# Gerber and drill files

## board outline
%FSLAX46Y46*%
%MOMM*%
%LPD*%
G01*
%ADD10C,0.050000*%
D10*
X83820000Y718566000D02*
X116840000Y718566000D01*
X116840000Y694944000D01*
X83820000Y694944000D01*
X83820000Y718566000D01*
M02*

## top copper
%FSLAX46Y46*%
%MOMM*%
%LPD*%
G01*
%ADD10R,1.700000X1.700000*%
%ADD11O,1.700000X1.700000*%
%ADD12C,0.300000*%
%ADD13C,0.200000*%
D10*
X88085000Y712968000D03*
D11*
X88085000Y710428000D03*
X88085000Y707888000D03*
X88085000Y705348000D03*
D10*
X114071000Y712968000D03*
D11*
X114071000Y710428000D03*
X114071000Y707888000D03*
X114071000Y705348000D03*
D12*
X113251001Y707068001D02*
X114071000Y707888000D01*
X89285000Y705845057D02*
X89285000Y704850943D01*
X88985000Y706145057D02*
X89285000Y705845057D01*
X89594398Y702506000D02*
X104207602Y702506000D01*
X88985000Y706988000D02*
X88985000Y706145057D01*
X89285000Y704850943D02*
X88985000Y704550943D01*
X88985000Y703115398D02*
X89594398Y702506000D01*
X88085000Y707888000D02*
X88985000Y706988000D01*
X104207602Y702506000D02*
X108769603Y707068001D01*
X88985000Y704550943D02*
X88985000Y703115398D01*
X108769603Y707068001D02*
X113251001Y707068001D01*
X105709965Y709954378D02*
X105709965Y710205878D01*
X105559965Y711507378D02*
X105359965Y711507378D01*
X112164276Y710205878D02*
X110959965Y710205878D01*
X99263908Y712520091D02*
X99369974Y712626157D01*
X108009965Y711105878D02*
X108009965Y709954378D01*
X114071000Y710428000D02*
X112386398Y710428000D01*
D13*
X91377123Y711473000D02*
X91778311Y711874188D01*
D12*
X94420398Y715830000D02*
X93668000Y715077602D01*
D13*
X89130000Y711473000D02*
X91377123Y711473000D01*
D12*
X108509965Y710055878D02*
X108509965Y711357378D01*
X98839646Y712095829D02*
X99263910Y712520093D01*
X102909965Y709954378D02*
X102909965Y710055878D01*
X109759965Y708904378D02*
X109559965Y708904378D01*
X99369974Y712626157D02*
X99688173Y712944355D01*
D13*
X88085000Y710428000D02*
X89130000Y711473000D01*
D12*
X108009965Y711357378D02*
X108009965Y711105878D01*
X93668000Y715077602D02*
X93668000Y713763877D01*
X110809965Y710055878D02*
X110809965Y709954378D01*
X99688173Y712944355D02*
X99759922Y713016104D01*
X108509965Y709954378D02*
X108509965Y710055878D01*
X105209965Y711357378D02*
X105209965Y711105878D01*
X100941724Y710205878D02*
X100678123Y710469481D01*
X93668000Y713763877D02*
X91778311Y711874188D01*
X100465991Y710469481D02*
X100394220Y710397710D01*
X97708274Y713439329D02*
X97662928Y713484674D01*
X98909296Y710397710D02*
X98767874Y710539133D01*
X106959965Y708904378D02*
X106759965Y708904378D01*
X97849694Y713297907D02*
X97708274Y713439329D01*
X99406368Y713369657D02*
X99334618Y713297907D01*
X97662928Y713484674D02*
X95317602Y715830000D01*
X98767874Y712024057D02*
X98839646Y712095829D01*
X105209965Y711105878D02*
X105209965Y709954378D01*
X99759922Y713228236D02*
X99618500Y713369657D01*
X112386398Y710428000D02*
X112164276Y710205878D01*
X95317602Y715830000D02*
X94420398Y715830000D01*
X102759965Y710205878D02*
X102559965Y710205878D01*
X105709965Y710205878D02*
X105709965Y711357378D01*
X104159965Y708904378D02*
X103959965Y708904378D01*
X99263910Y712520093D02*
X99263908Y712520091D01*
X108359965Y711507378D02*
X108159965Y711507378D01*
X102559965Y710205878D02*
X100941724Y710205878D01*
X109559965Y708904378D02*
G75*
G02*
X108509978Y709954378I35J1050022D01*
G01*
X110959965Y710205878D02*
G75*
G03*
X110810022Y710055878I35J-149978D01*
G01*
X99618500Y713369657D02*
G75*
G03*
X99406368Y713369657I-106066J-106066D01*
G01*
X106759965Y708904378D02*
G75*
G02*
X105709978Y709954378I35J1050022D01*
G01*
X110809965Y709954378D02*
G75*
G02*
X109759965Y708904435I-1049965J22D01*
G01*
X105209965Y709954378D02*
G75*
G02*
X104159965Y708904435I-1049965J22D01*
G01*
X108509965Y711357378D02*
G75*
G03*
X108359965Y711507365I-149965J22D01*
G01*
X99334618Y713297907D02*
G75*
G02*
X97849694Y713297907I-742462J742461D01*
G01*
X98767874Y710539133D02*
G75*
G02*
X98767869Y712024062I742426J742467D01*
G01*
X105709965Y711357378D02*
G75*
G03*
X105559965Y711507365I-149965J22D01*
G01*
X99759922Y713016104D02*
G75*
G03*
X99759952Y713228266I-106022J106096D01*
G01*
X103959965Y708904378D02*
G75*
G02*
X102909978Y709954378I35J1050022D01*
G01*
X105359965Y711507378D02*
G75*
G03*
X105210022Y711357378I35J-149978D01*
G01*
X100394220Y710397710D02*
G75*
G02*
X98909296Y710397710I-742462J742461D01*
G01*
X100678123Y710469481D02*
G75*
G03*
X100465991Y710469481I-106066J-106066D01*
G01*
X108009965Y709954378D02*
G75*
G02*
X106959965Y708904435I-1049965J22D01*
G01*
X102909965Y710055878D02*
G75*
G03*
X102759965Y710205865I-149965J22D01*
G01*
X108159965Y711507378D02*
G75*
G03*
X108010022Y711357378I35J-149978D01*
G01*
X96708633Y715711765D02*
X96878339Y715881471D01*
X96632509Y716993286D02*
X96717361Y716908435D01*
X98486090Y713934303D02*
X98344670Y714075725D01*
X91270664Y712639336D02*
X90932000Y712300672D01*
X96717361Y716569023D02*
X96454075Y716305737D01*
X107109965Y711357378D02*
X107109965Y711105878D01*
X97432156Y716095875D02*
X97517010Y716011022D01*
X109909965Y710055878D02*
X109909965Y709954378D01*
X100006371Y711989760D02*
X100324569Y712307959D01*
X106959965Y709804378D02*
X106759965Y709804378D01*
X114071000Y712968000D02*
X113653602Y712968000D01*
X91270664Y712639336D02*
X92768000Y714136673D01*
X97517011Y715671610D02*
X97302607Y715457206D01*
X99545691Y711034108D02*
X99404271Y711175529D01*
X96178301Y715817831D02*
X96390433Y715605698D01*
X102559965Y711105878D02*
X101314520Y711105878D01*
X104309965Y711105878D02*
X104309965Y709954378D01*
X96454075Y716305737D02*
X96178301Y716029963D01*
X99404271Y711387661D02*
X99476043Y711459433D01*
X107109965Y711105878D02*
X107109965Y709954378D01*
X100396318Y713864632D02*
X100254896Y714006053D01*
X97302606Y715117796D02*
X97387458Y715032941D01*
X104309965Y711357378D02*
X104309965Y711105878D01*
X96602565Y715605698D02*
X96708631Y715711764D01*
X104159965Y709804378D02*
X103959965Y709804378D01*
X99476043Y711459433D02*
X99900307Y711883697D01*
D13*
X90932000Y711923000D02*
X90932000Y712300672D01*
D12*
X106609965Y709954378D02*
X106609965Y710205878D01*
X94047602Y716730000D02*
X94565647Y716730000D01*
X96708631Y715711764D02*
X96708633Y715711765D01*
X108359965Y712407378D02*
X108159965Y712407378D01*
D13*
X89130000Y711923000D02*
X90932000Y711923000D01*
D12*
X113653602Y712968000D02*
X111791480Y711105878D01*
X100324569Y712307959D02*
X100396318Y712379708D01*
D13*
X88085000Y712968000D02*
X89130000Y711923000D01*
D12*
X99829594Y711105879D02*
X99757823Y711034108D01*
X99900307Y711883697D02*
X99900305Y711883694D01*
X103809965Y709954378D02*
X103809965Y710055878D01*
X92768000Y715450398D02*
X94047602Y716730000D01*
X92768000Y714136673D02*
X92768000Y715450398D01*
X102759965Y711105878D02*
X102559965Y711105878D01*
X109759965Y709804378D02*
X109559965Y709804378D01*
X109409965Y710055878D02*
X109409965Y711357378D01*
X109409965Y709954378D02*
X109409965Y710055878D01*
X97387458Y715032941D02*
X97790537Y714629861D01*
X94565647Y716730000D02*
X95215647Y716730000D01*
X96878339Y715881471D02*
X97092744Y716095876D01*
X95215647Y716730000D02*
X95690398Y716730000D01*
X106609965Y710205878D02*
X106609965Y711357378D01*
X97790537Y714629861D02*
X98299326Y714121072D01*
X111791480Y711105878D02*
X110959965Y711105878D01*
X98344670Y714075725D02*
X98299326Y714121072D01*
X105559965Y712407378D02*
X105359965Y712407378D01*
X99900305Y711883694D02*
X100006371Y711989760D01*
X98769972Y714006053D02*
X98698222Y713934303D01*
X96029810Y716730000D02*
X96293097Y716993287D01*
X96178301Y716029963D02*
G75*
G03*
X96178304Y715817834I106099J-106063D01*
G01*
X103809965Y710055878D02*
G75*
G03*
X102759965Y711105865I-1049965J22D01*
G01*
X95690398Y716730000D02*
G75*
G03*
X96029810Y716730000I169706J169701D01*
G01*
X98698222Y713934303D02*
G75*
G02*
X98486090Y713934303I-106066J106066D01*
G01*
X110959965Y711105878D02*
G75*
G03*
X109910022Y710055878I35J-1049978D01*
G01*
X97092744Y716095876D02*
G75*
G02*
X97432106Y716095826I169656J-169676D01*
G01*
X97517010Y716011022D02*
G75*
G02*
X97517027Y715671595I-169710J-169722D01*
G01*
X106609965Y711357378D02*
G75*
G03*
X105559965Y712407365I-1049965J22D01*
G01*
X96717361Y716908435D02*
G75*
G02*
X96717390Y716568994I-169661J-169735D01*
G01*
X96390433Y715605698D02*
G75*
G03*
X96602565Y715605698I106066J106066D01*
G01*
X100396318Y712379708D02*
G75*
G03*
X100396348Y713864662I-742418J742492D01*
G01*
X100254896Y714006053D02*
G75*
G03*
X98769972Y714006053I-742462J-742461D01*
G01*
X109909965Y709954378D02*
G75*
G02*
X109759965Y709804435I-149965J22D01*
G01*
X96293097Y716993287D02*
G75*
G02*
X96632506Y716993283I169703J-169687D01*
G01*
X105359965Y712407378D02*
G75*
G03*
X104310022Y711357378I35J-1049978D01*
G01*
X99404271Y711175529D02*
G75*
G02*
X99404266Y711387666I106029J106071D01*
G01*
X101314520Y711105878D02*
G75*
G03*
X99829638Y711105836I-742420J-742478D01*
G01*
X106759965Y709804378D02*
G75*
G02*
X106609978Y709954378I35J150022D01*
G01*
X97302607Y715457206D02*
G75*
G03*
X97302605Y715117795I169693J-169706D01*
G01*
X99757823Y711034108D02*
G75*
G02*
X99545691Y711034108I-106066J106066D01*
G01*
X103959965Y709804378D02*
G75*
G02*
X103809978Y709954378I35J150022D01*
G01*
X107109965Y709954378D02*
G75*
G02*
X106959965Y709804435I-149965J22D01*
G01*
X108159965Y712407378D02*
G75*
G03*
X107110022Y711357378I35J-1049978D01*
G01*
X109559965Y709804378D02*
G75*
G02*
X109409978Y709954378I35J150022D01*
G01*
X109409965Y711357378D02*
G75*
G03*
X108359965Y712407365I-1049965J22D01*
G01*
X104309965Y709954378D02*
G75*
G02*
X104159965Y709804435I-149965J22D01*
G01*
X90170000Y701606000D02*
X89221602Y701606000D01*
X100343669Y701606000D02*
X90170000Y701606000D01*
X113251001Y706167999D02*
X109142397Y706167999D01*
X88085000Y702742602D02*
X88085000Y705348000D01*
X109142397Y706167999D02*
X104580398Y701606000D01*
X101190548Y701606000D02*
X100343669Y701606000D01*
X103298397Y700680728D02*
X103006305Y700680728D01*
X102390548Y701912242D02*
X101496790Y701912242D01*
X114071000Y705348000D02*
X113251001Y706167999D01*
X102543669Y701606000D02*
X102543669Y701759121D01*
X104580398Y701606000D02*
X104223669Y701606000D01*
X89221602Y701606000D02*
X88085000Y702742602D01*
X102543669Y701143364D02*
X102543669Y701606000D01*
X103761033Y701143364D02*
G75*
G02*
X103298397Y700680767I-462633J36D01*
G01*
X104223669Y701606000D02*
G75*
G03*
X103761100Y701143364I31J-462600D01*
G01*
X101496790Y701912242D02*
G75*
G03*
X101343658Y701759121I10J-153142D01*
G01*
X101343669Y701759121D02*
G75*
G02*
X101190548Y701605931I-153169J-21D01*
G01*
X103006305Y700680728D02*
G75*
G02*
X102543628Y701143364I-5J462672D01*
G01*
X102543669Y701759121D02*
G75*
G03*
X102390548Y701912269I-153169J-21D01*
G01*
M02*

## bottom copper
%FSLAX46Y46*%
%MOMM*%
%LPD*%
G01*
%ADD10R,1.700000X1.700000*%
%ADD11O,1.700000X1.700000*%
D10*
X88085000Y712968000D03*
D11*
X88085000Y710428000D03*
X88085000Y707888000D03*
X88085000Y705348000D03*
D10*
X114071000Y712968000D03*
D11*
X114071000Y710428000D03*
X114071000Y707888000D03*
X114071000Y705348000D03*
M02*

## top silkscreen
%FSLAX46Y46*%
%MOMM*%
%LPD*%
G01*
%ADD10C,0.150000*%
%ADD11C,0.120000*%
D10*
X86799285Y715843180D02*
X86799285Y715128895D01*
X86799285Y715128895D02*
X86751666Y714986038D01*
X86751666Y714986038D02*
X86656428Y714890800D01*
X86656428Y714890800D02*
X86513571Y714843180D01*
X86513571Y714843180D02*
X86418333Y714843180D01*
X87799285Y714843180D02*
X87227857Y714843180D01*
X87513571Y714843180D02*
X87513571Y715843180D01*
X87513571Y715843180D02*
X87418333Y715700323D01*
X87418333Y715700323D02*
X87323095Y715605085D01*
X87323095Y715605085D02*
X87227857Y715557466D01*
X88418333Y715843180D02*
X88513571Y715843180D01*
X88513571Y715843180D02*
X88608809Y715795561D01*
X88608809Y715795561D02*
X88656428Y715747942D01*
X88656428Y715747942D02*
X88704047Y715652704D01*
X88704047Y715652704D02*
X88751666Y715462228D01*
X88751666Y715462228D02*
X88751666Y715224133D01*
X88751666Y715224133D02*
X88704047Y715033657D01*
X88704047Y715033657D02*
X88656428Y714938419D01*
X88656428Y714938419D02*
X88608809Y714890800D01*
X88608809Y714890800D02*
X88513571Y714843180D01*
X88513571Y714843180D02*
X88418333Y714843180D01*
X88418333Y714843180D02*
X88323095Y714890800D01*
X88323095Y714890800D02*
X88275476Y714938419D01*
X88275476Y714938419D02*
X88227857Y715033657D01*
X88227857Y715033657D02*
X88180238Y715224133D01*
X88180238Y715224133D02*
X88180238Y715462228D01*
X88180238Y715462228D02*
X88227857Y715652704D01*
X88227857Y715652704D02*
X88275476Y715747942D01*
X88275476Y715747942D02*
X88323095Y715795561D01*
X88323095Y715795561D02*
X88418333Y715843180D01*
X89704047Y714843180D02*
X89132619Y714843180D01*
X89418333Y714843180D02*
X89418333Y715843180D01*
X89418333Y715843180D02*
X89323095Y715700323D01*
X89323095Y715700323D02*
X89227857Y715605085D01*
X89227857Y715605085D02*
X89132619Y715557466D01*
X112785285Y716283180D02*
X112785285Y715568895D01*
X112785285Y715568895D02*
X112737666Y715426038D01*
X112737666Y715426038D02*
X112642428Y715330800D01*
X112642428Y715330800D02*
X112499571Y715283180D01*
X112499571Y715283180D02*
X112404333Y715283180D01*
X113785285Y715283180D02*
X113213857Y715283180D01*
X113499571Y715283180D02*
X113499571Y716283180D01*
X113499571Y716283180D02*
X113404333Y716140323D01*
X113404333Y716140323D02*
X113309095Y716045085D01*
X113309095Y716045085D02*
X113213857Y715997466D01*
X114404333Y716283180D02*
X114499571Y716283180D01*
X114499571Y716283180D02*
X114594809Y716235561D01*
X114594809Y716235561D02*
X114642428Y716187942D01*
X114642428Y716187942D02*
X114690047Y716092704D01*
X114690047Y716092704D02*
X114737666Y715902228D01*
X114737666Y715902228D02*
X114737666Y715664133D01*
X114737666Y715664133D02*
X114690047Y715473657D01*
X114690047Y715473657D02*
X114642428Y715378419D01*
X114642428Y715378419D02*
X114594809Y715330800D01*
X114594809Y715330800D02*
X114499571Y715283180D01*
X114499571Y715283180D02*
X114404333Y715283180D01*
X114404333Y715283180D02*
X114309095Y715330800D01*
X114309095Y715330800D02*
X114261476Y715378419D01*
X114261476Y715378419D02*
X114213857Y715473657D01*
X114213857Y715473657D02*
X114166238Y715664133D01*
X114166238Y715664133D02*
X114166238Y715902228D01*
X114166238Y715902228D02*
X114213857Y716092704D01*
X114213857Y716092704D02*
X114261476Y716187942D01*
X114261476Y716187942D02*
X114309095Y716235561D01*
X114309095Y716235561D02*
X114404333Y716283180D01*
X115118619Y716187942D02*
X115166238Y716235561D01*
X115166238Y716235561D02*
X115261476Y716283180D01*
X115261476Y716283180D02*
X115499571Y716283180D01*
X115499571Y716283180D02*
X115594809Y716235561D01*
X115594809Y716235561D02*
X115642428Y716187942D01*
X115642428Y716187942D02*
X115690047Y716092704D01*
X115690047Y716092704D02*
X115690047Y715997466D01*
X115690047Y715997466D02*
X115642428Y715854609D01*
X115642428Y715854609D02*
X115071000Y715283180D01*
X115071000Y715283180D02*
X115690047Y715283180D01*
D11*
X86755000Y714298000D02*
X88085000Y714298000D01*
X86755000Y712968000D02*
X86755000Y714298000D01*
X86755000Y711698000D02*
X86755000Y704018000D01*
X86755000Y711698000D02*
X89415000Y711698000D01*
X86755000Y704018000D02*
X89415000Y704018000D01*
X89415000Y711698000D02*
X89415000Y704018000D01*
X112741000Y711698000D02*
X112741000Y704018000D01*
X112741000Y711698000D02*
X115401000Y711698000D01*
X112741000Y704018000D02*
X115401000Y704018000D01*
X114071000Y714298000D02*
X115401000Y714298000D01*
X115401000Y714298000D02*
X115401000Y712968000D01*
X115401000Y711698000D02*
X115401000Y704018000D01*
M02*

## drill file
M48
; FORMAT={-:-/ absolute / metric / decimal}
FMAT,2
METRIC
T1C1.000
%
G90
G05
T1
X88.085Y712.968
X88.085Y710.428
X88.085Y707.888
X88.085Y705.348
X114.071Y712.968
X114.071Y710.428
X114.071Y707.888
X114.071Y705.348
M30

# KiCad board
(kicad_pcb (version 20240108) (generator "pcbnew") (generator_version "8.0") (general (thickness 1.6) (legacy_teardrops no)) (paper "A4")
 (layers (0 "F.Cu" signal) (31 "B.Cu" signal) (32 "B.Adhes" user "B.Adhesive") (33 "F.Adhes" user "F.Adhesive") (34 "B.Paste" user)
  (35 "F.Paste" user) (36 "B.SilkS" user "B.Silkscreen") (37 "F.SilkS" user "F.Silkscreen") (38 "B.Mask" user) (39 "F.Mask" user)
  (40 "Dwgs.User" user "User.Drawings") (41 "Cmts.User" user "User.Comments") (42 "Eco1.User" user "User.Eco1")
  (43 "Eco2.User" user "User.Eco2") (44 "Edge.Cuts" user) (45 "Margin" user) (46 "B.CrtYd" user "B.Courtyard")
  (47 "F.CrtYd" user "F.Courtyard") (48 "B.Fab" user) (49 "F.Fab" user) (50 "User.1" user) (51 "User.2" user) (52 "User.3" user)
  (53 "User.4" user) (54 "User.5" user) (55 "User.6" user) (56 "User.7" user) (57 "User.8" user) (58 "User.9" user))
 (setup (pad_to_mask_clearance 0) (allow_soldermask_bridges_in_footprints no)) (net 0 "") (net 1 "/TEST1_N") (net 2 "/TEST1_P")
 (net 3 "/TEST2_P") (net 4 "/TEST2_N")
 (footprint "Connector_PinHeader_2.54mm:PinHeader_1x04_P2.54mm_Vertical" (layer "F.Cu") (at 88.085 -712.968)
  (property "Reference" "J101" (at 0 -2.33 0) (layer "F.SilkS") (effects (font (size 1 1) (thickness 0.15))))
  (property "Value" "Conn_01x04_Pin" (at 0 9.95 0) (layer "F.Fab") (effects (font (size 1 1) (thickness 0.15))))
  (fp_line (start -1.33 -1.33) (end 0 -1.33) (stroke (width 0.12) (type solid)) (layer "F.SilkS"))
  (fp_line (start -1.33 0) (end -1.33 -1.33) (stroke (width 0.12) (type solid)) (layer "F.SilkS"))
  (fp_line (start -1.33 1.27) (end -1.33 8.95) (stroke (width 0.12) (type solid)) (layer "F.SilkS"))
  (fp_line (start -1.33 1.27) (end 1.33 1.27) (stroke (width 0.12) (type solid)) (layer "F.SilkS"))
  (fp_line (start -1.33 8.95) (end 1.33 8.95) (stroke (width 0.12) (type solid)) (layer "F.SilkS"))
  (fp_line (start 1.33 1.27) (end 1.33 8.95) (stroke (width 0.12) (type solid)) (layer "F.SilkS"))
  (pad "1" thru_hole rect (at 0 0) (size 1.7 1.7) (drill 1) (layers "*.Cu" "*.Mask") (remove_unused_layers no) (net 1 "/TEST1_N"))
  (pad "2" thru_hole oval (at 0 2.54) (size 1.7 1.7) (drill 1) (layers "*.Cu" "*.Mask") (remove_unused_layers no) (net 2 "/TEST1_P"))
  (pad "3" thru_hole oval (at 0 5.08) (size 1.7 1.7) (drill 1) (layers "*.Cu" "*.Mask") (remove_unused_layers no) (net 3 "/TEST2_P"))
  (pad "4" thru_hole oval (at 0 7.62) (size 1.7 1.7) (drill 1) (layers "*.Cu" "*.Mask") (remove_unused_layers no) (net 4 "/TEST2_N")))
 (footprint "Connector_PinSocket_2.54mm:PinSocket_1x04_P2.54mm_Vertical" (layer "F.Cu") (at 114.071 -712.968)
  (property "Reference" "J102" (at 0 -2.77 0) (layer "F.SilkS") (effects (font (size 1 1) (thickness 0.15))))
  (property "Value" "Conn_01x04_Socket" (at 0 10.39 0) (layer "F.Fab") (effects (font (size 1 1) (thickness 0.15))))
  (fp_line (start -1.33 1.27) (end -1.33 8.95) (stroke (width 0.12) (type solid)) (layer "F.SilkS"))
  (fp_line (start -1.33 1.27) (end 1.33 1.27) (stroke (width 0.12) (type solid)) (layer "F.SilkS"))
  (fp_line (start -1.33 8.95) (end 1.33 8.95) (stroke (width 0.12) (type solid)) (layer "F.SilkS"))
  (fp_line (start 0 -1.33) (end 1.33 -1.33) (stroke (width 0.12) (type solid)) (layer "F.SilkS"))
  (fp_line (start 1.33 -1.33) (end 1.33 0) (stroke (width 0.12) (type solid)) (layer "F.SilkS"))
  (fp_line (start 1.33 1.27) (end 1.33 8.95) (stroke (width 0.12) (type solid)) (layer "F.SilkS"))
  (pad "1" thru_hole rect (at 0 0) (size 1.7 1.7) (drill 1) (layers "*.Cu" "*.Mask") (remove_unused_layers no) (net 1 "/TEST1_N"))
  (pad "2" thru_hole oval (at 0 2.54) (size 1.7 1.7) (drill 1) (layers "*.Cu" "*.Mask") (remove_unused_layers no) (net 2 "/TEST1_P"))
  (pad "3" thru_hole oval (at 0 5.08) (size 1.7 1.7) (drill 1) (layers "*.Cu" "*.Mask") (remove_unused_layers no) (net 3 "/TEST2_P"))
  (pad "4" thru_hole oval (at 0 7.62) (size 1.7 1.7) (drill 1) (layers "*.Cu" "*.Mask") (remove_unused_layers no) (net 4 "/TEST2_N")))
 (gr_rect (start 83.82 -718.566) (end 116.84 -694.944) (stroke (width 0.05) (type default)) (fill none) (layer "Edge.Cuts"))
 (segment (start 113.251001 -707.068001) (end 114.071 -707.888) (width 0.3) (layer "F.Cu") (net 3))
 (segment (start 89.285 -705.845057) (end 89.285 -704.850943) (width 0.3) (layer "F.Cu") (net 3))
 (segment (start 88.985 -706.145057) (end 89.285 -705.845057) (width 0.3) (layer "F.Cu") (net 3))
 (segment (start 89.594398 -702.506) (end 104.207602 -702.506) (width 0.3) (layer "F.Cu") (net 3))
 (segment (start 88.985 -706.988) (end 88.985 -706.145057) (width 0.3) (layer "F.Cu") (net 3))
 (segment (start 89.285 -704.850943) (end 88.985 -704.550943) (width 0.3) (layer "F.Cu") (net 3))
 (segment (start 88.985 -703.115398) (end 89.594398 -702.506) (width 0.3) (layer "F.Cu") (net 3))
 (segment (start 88.085 -707.888) (end 88.985 -706.988) (width 0.3) (layer "F.Cu") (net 3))
 (segment (start 104.207602 -702.506) (end 108.769603 -707.068001) (width 0.3) (layer "F.Cu") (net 3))
 (segment (start 88.985 -704.550943) (end 88.985 -703.115398) (width 0.3) (layer "F.Cu") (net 3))
 (segment (start 108.769603 -707.068001) (end 113.251001 -707.068001) (width 0.3) (layer "F.Cu") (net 3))
 (segment (start 105.709965 -709.954378) (end 105.709965 -710.205878) (width 0.3) (layer "F.Cu") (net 2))
 (segment (start 105.559965 -711.507378) (end 105.359965 -711.507378) (width 0.3) (layer "F.Cu") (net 2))
 (segment (start 112.164276 -710.205878) (end 110.959965 -710.205878) (width 0.3) (layer "F.Cu") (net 2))
 (segment (start 99.263908 -712.520091) (end 99.369974 -712.626157) (width 0.3) (layer "F.Cu") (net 2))
 (segment (start 108.009965 -711.105878) (end 108.009965 -709.954378) (width 0.3) (layer "F.Cu") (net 2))
 (segment (start 114.071 -710.428) (end 112.386398 -710.428) (width 0.3) (layer "F.Cu") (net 2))
 (segment (start 91.377123 -711.473) (end 91.778311 -711.874188) (width 0.2) (layer "F.Cu") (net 2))
 (segment (start 94.420398 -715.83) (end 93.668 -715.077602) (width 0.3) (layer "F.Cu") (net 2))
 (segment (start 89.13 -711.473) (end 91.377123 -711.473) (width 0.2) (layer "F.Cu") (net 2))
 (segment (start 108.509965 -710.055878) (end 108.509965 -711.357378) (width 0.3) (layer "F.Cu") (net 2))
 (segment (start 98.839646 -712.095829) (end 99.26391 -712.520093) (width 0.3) (layer "F.Cu") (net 2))
 (segment (start 102.909965 -709.954378) (end 102.909965 -710.055878) (width 0.3) (layer "F.Cu") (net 2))
 (segment (start 109.759965 -708.904378) (end 109.559965 -708.904378) (width 0.3) (layer "F.Cu") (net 2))
 (segment (start 99.369974 -712.626157) (end 99.688173 -712.944355) (width 0.3) (layer "F.Cu") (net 2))
 (segment (start 88.085 -710.428) (end 89.13 -711.473) (width 0.2) (layer "F.Cu") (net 2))
 (segment (start 108.009965 -711.357378) (end 108.009965 -711.105878) (width 0.3) (layer "F.Cu") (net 2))
 (segment (start 93.668 -715.077602) (end 93.668 -713.763877) (width 0.3) (layer "F.Cu") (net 2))
 (segment (start 110.809965 -710.055878) (end 110.809965 -709.954378) (width 0.3) (layer "F.Cu") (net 2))
 (segment (start 99.688173 -712.944355) (end 99.759922 -713.016104) (width 0.3) (layer "F.Cu") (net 2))
 (segment (start 108.509965 -709.954378) (end 108.509965 -710.055878) (width 0.3) (layer "F.Cu") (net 2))
 (segment (start 105.209965 -711.357378) (end 105.209965 -711.105878) (width 0.3) (layer "F.Cu") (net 2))
 (segment (start 100.941724 -710.205878) (end 100.678123 -710.469481) (width 0.3) (layer "F.Cu") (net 2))
 (segment (start 93.668 -713.763877) (end 91.778311 -711.874188) (width 0.3) (layer "F.Cu") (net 2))
 (segment (start 100.465991 -710.469481) (end 100.39422 -710.39771) (width 0.3) (layer "F.Cu") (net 2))
 (segment (start 97.708274 -713.439329) (end 97.662928 -713.484674) (width 0.3) (layer "F.Cu") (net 2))
 (segment (start 98.909296 -710.39771) (end 98.767874 -710.539133) (width 0.3) (layer "F.Cu") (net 2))
 (segment (start 106.959965 -708.904378) (end 106.759965 -708.904378) (width 0.3) (layer "F.Cu") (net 2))
 (segment (start 97.849694 -713.297907) (end 97.708274 -713.439329) (width 0.3) (layer "F.Cu") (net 2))
 (segment (start 99.406368 -713.369657) (end 99.334618 -713.297907) (width 0.3) (layer "F.Cu") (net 2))
 (segment (start 97.662928 -713.484674) (end 95.317602 -715.83) (width 0.3) (layer "F.Cu") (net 2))
 (segment (start 98.767874 -712.024057) (end 98.839646 -712.095829) (width 0.3) (layer "F.Cu") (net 2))
 (segment (start 105.209965 -711.105878) (end 105.209965 -709.954378) (width 0.3) (layer "F.Cu") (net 2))
 (segment (start 99.759922 -713.228236) (end 99.6185 -713.369657) (width 0.3) (layer "F.Cu") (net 2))
 (segment (start 112.386398 -710.428) (end 112.164276 -710.205878) (width 0.3) (layer "F.Cu") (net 2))
 (segment (start 95.317602 -715.83) (end 94.420398 -715.83) (width 0.3) (layer "F.Cu") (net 2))
 (segment (start 102.759965 -710.205878) (end 102.559965 -710.205878) (width 0.3) (layer "F.Cu") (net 2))
 (segment (start 105.709965 -710.205878) (end 105.709965 -711.357378) (width 0.3) (layer "F.Cu") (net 2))
 (segment (start 104.159965 -708.904378) (end 103.959965 -708.904378) (width 0.3) (layer "F.Cu") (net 2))
 (segment (start 99.26391 -712.520093) (end 99.263908 -712.520091) (width 0.3) (layer "F.Cu") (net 2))
 (segment (start 108.359965 -711.507378) (end 108.159965 -711.507378) (width 0.3) (layer "F.Cu") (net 2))
 (segment (start 102.559965 -710.205878) (end 100.941724 -710.205878) (width 0.3) (layer "F.Cu") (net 2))
 (arc (start 109.559965 -708.904378) (mid 108.817503 -709.211916) (end 108.509965 -709.954378) (width 0.3) (layer "F.Cu") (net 2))
 (arc (start 110.959965 -710.205878) (mid 110.853899 -710.161944) (end 110.809965 -710.055878) (width 0.3) (layer "F.Cu") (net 2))
 (arc (start 99.6185 -713.369657) (mid 99.512434 -713.413591) (end 99.406368 -713.369657) (width 0.3) (layer "F.Cu") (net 2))
 (arc (start 106.759965 -708.904378) (mid 106.017503 -709.211916) (end 105.709965 -709.954378) (width 0.3) (layer "F.Cu") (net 2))
 (arc (start 110.809965 -709.954378) (mid 110.502427 -709.211916) (end 109.759965 -708.904378) (width 0.3) (layer "F.Cu") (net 2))
 (arc (start 105.209965 -709.954378) (mid 104.902427 -709.211916) (end 104.159965 -708.904378) (width 0.3) (layer "F.Cu") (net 2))
 (arc (start 108.509965 -711.357378) (mid 108.466031 -711.463444) (end 108.359965 -711.507378) (width 0.3) (layer "F.Cu") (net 2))
 (arc (start 99.334618 -713.297907) (mid 98.592156 -712.990369) (end 97.849694 -713.297907) (width 0.3) (layer "F.Cu") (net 2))
 (arc (start 98.767874 -710.539133) (mid 98.460336 -711.281595) (end 98.767874 -712.024057) (width 0.3) (layer "F.Cu") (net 2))
 (arc (start 105.709965 -711.357378) (mid 105.666031 -711.463444) (end 105.559965 -711.507378) (width 0.3) (layer "F.Cu") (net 2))
 (arc (start 99.759922 -713.016104) (mid 99.803856 -713.12217) (end 99.759922 -713.228236) (width 0.3) (layer "F.Cu") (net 2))
 (arc (start 103.959965 -708.904378) (mid 103.217503 -709.211916) (end 102.909965 -709.954378) (width 0.3) (layer "F.Cu") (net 2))
 (arc (start 105.359965 -711.507378) (mid 105.253899 -711.463444) (end 105.209965 -711.357378) (width 0.3) (layer "F.Cu") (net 2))
 (arc (start 100.39422 -710.39771) (mid 99.651758 -710.090172) (end 98.909296 -710.39771) (width 0.3) (layer "F.Cu") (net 2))
 (arc (start 100.678123 -710.469481) (mid 100.572057 -710.513415) (end 100.465991 -710.469481) (width 0.3) (layer "F.Cu") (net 2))
 (arc (start 108.009965 -709.954378) (mid 107.702427 -709.211916) (end 106.959965 -708.904378) (width 0.3) (layer "F.Cu") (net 2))
 (arc (start 102.909965 -710.055878) (mid 102.866031 -710.161944) (end 102.759965 -710.205878) (width 0.3) (layer "F.Cu") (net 2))
 (arc (start 108.159965 -711.507378) (mid 108.053899 -711.463444) (end 108.009965 -711.357378) (width 0.3) (layer "F.Cu") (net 2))
 (segment (start 96.708633 -715.711765) (end 96.878339 -715.881471) (width 0.3) (layer "F.Cu") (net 1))
 (segment (start 96.632509 -716.993286) (end 96.717361 -716.908435) (width 0.3) (layer "F.Cu") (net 1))
 (segment (start 98.48609 -713.934303) (end 98.34467 -714.075725) (width 0.3) (layer "F.Cu") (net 1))
 (segment (start 91.270664 -712.639336) (end 90.932 -712.300672) (width 0.3) (layer "F.Cu") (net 1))
 (segment (start 96.717361 -716.569023) (end 96.454075 -716.305737) (width 0.3) (layer "F.Cu") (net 1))
 (segment (start 107.109965 -711.357378) (end 107.109965 -711.105878) (width 0.3) (layer "F.Cu") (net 1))
 (segment (start 97.432156 -716.095875) (end 97.51701 -716.011022) (width 0.3) (layer "F.Cu") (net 1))
 (segment (start 109.909965 -710.055878) (end 109.909965 -709.954378) (width 0.3) (layer "F.Cu") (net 1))
 (segment (start 100.006371 -711.98976) (end 100.324569 -712.307959) (width 0.3) (layer "F.Cu") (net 1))
 (segment (start 106.959965 -709.804378) (end 106.759965 -709.804378) (width 0.3) (layer "F.Cu") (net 1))
 (segment (start 114.071 -712.968) (end 113.653602 -712.968) (width 0.3) (layer "F.Cu") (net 1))
 (segment (start 91.270664 -712.639336) (end 92.768 -714.136673) (width 0.3) (layer "F.Cu") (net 1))
 (segment (start 97.517011 -715.67161) (end 97.302607 -715.457206) (width 0.3) (layer "F.Cu") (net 1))
 (segment (start 99.545691 -711.034108) (end 99.404271 -711.175529) (width 0.3) (layer "F.Cu") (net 1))
 (segment (start 96.178301 -715.817831) (end 96.390433 -715.605698) (width 0.3) (layer "F.Cu") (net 1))
 (segment (start 102.559965 -711.105878) (end 101.31452 -711.105878) (width 0.3) (layer "F.Cu") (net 1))
 (segment (start 104.309965 -711.105878) (end 104.309965 -709.954378) (width 0.3) (layer "F.Cu") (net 1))
 (segment (start 96.454075 -716.305737) (end 96.178301 -716.029963) (width 0.3) (layer "F.Cu") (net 1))
 (segment (start 99.404271 -711.387661) (end 99.476043 -711.459433) (width 0.3) (layer "F.Cu") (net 1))
 (segment (start 107.109965 -711.105878) (end 107.109965 -709.954378) (width 0.3) (layer "F.Cu") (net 1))
 (segment (start 100.396318 -713.864632) (end 100.254896 -714.006053) (width 0.3) (layer "F.Cu") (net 1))
 (segment (start 97.302606 -715.117796) (end 97.387458 -715.032941) (width 0.3) (layer "F.Cu") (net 1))
 (segment (start 104.309965 -711.357378) (end 104.309965 -711.105878) (width 0.3) (layer "F.Cu") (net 1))
 (segment (start 96.602565 -715.605698) (end 96.708631 -715.711764) (width 0.3) (layer "F.Cu") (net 1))
 (segment (start 104.159965 -709.804378) (end 103.959965 -709.804378) (width 0.3) (layer "F.Cu") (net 1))
 (segment (start 99.476043 -711.459433) (end 99.900307 -711.883697) (width 0.3) (layer "F.Cu") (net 1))
 (segment (start 90.932 -711.923) (end 90.932 -712.300672) (width 0.2) (layer "F.Cu") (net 1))
 (segment (start 106.609965 -709.954378) (end 106.609965 -710.205878) (width 0.3) (layer "F.Cu") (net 1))
 (segment (start 94.047602 -716.73) (end 94.565647 -716.73) (width 0.3) (layer "F.Cu") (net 1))
 (segment (start 96.708631 -715.711764) (end 96.708633 -715.711765) (width 0.3) (layer "F.Cu") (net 1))
 (segment (start 108.359965 -712.407378) (end 108.159965 -712.407378) (width 0.3) (layer "F.Cu") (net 1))
 (segment (start 89.13 -711.923) (end 90.932 -711.923) (width 0.2) (layer "F.Cu") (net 1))
 (segment (start 113.653602 -712.968) (end 111.79148 -711.105878) (width 0.3) (layer "F.Cu") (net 1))
 (segment (start 100.324569 -712.307959) (end 100.396318 -712.379708) (width 0.3) (layer "F.Cu") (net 1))
 (segment (start 88.085 -712.968) (end 89.13 -711.923) (width 0.2) (layer "F.Cu") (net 1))
 (segment (start 99.829594 -711.105879) (end 99.757823 -711.034108) (width 0.3) (layer "F.Cu") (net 1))
 (segment (start 99.900307 -711.883697) (end 99.900305 -711.883694) (width 0.3) (layer "F.Cu") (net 1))
 (segment (start 103.809965 -709.954378) (end 103.809965 -710.055878) (width 0.3) (layer "F.Cu") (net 1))
 (segment (start 92.768 -715.450398) (end 94.047602 -716.73) (width 0.3) (layer "F.Cu") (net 1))
 (segment (start 92.768 -714.136673) (end 92.768 -715.450398) (width 0.3) (layer "F.Cu") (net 1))
 (segment (start 102.759965 -711.105878) (end 102.559965 -711.105878) (width 0.3) (layer "F.Cu") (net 1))
 (segment (start 109.759965 -709.804378) (end 109.559965 -709.804378) (width 0.3) (layer "F.Cu") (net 1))
 (segment (start 109.409965 -710.055878) (end 109.409965 -711.357378) (width 0.3) (layer "F.Cu") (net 1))
 (segment (start 109.409965 -709.954378) (end 109.409965 -710.055878) (width 0.3) (layer "F.Cu") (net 1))
 (segment (start 97.387458 -715.032941) (end 97.790537 -714.629861) (width 0.3) (layer "F.Cu") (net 1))
 (segment (start 94.565647 -716.73) (end 95.215647 -716.73) (width 0.3) (layer "F.Cu") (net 1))
 (segment (start 96.878339 -715.881471) (end 97.092744 -716.095876) (width 0.3) (layer "F.Cu") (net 1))
 (segment (start 95.215647 -716.73) (end 95.690398 -716.73) (width 0.3) (layer "F.Cu") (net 1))
 (segment (start 106.609965 -710.205878) (end 106.609965 -711.357378) (width 0.3) (layer "F.Cu") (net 1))
 (segment (start 97.790537 -714.629861) (end 98.299326 -714.121072) (width 0.3) (layer "F.Cu") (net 1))
 (segment (start 111.79148 -711.105878) (end 110.959965 -711.105878) (width 0.3) (layer "F.Cu") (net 1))
 (segment (start 98.34467 -714.075725) (end 98.299326 -714.121072) (width 0.3) (layer "F.Cu") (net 1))
 (segment (start 105.559965 -712.407378) (end 105.359965 -712.407378) (width 0.3) (layer "F.Cu") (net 1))
 (segment (start 99.900305 -711.883694) (end 100.006371 -711.98976) (width 0.3) (layer "F.Cu") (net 1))
 (segment (start 98.769972 -714.006053) (end 98.698222 -713.934303) (width 0.3) (layer "F.Cu") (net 1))
 (segment (start 96.02981 -716.73) (end 96.293097 -716.993287) (width 0.3) (layer "F.Cu") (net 1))
 (arc (start 96.178301 -716.029963) (mid 96.134367 -715.923897) (end 96.178301 -715.817831) (width 0.3) (layer "F.Cu") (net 1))
 (arc (start 103.809965 -710.055878) (mid 103.502427 -710.79834) (end 102.759965 -711.105878) (width 0.3) (layer "F.Cu") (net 1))
 (arc (start 95.690398 -716.73) (mid 95.860105 -716.659704) (end 96.02981 -716.73) (width 0.3) (layer "F.Cu") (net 1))
 (arc (start 98.698222 -713.934303) (mid 98.592156 -713.890369) (end 98.48609 -713.934303) (width 0.3) (layer "F.Cu") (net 1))
 (arc (start 110.959965 -711.105878) (mid 110.217503 -710.79834) (end 109.909965 -710.055878) (width 0.3) (layer "F.Cu") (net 1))
 (arc (start 97.092744 -716.095876) (mid 97.262449 -716.166171) (end 97.432156 -716.095875) (width 0.3) (layer "F.Cu") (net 1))
 (arc (start 97.51701 -716.011022) (mid 97.587305 -715.841316) (end 97.517011 -715.67161) (width 0.3) (layer "F.Cu") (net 1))
 (arc (start 106.609965 -711.357378) (mid 106.302427 -712.09984) (end 105.559965 -712.407378) (width 0.3) (layer "F.Cu") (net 1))
 (arc (start 96.717361 -716.908435) (mid 96.787657 -716.738728) (end 96.717361 -716.569023) (width 0.3) (layer "F.Cu") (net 1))
 (arc (start 96.390433 -715.605698) (mid 96.496499 -715.561764) (end 96.602565 -715.605698) (width 0.3) (layer "F.Cu") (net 1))
 (arc (start 100.396318 -712.379708) (mid 100.703856 -713.12217) (end 100.396318 -713.864632) (width 0.3) (layer "F.Cu") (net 1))
 (arc (start 100.254896 -714.006053) (mid 99.512434 -714.313591) (end 98.769972 -714.006053) (width 0.3) (layer "F.Cu") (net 1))
 (arc (start 109.909965 -709.954378) (mid 109.866031 -709.848312) (end 109.759965 -709.804378) (width 0.3) (layer "F.Cu") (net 1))
 (arc (start 96.293097 -716.993287) (mid 96.462802 -717.063582) (end 96.632509 -716.993286) (width 0.3) (layer "F.Cu") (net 1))
 (arc (start 105.359965 -712.407378) (mid 104.617503 -712.09984) (end 104.309965 -711.357378) (width 0.3) (layer "F.Cu") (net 1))
 (arc (start 99.404271 -711.175529) (mid 99.360337 -711.281595) (end 99.404271 -711.387661) (width 0.3) (layer "F.Cu") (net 1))
 (arc (start 101.31452 -711.105878) (mid 100.572058 -711.413416) (end 99.829594 -711.105879) (width 0.3) (layer "F.Cu") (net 1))
 (arc (start 106.759965 -709.804378) (mid 106.653899 -709.848312) (end 106.609965 -709.954378) (width 0.3) (layer "F.Cu") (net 1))
 (arc (start 97.302607 -715.457206) (mid 97.232313 -715.2875) (end 97.302606 -715.117796) (width 0.3) (layer "F.Cu") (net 1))
 (arc (start 99.757823 -711.034108) (mid 99.651757 -710.990174) (end 99.545691 -711.034108) (width 0.3) (layer "F.Cu") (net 1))
 (arc (start 103.959965 -709.804378) (mid 103.853899 -709.848312) (end 103.809965 -709.954378) (width 0.3) (layer "F.Cu") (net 1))
 (arc (start 107.109965 -709.954378) (mid 107.066031 -709.848312) (end 106.959965 -709.804378) (width 0.3) (layer "F.Cu") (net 1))
 (arc (start 108.159965 -712.407378) (mid 107.417503 -712.09984) (end 107.109965 -711.357378) (width 0.3) (layer "F.Cu") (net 1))
 (arc (start 109.559965 -709.804378) (mid 109.453899 -709.848312) (end 109.409965 -709.954378) (width 0.3) (layer "F.Cu") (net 1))
 (arc (start 109.409965 -711.357378) (mid 109.102427 -712.09984) (end 108.359965 -712.407378) (width 0.3) (layer "F.Cu") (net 1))
 (arc (start 104.309965 -709.954378) (mid 104.266031 -709.848312) (end 104.159965 -709.804378) (width 0.3) (layer "F.Cu") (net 1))
 (segment (start 90.17 -701.606) (end 89.221602 -701.606) (width 0.3) (layer "F.Cu") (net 4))
 (segment (start 100.343669 -701.606) (end 90.17 -701.606) (width 0.3) (layer "F.Cu") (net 4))
 (segment (start 113.251001 -706.167999) (end 109.142397 -706.167999) (width 0.3) (layer "F.Cu") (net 4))
 (segment (start 88.085 -702.742602) (end 88.085 -705.348) (width 0.3) (layer "F.Cu") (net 4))
 (segment (start 109.142397 -706.167999) (end 104.580398 -701.606) (width 0.3) (layer "F.Cu") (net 4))
 (segment (start 101.190548 -701.606) (end 100.343669 -701.606) (width 0.3) (layer "F.Cu") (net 4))
 (segment (start 103.298397 -700.680728) (end 103.006305 -700.680728) (width 0.3) (layer "F.Cu") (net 4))
 (segment (start 102.390548 -701.912242) (end 101.49679 -701.912242) (width 0.3) (layer "F.Cu") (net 4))
 (segment (start 114.071 -705.348) (end 113.251001 -706.167999) (width 0.3) (layer "F.Cu") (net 4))
 (segment (start 102.543669 -701.606) (end 102.543669 -701.759121) (width 0.3) (layer "F.Cu") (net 4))
 (segment (start 104.580398 -701.606) (end 104.223669 -701.606) (width 0.3) (layer "F.Cu") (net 4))
 (segment (start 89.221602 -701.606) (end 88.085 -702.742602) (width 0.3) (layer "F.Cu") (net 4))
 (segment (start 102.543669 -701.143364) (end 102.543669 -701.606) (width 0.3) (layer "F.Cu") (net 4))
 (arc (start 103.761033 -701.143364) (mid 103.62553 -700.816231) (end 103.298397 -700.680728) (width 0.3) (layer "F.Cu") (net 4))
 (arc (start 104.223669 -701.606) (mid 103.896536 -701.470497) (end 103.761033 -701.143364) (width 0.3) (layer "F.Cu") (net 4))
 (arc (start 101.49679 -701.912242) (mid 101.388517 -701.867394) (end 101.343669 -701.759121) (width 0.3) (layer "F.Cu") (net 4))
 (arc (start 101.343669 -701.759121) (mid 101.298821 -701.650848) (end 101.190548 -701.606) (width 0.3) (layer "F.Cu") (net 4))
 (arc (start 103.006305 -700.680728) (mid 102.679172 -700.816231) (end 102.543669 -701.143364) (width 0.3) (layer "F.Cu") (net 4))
 (arc (start 102.543669 -701.759121) (mid 102.498821 -701.867394) (end 102.390548 -701.912242) (width 0.3) (layer "F.Cu") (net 4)))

